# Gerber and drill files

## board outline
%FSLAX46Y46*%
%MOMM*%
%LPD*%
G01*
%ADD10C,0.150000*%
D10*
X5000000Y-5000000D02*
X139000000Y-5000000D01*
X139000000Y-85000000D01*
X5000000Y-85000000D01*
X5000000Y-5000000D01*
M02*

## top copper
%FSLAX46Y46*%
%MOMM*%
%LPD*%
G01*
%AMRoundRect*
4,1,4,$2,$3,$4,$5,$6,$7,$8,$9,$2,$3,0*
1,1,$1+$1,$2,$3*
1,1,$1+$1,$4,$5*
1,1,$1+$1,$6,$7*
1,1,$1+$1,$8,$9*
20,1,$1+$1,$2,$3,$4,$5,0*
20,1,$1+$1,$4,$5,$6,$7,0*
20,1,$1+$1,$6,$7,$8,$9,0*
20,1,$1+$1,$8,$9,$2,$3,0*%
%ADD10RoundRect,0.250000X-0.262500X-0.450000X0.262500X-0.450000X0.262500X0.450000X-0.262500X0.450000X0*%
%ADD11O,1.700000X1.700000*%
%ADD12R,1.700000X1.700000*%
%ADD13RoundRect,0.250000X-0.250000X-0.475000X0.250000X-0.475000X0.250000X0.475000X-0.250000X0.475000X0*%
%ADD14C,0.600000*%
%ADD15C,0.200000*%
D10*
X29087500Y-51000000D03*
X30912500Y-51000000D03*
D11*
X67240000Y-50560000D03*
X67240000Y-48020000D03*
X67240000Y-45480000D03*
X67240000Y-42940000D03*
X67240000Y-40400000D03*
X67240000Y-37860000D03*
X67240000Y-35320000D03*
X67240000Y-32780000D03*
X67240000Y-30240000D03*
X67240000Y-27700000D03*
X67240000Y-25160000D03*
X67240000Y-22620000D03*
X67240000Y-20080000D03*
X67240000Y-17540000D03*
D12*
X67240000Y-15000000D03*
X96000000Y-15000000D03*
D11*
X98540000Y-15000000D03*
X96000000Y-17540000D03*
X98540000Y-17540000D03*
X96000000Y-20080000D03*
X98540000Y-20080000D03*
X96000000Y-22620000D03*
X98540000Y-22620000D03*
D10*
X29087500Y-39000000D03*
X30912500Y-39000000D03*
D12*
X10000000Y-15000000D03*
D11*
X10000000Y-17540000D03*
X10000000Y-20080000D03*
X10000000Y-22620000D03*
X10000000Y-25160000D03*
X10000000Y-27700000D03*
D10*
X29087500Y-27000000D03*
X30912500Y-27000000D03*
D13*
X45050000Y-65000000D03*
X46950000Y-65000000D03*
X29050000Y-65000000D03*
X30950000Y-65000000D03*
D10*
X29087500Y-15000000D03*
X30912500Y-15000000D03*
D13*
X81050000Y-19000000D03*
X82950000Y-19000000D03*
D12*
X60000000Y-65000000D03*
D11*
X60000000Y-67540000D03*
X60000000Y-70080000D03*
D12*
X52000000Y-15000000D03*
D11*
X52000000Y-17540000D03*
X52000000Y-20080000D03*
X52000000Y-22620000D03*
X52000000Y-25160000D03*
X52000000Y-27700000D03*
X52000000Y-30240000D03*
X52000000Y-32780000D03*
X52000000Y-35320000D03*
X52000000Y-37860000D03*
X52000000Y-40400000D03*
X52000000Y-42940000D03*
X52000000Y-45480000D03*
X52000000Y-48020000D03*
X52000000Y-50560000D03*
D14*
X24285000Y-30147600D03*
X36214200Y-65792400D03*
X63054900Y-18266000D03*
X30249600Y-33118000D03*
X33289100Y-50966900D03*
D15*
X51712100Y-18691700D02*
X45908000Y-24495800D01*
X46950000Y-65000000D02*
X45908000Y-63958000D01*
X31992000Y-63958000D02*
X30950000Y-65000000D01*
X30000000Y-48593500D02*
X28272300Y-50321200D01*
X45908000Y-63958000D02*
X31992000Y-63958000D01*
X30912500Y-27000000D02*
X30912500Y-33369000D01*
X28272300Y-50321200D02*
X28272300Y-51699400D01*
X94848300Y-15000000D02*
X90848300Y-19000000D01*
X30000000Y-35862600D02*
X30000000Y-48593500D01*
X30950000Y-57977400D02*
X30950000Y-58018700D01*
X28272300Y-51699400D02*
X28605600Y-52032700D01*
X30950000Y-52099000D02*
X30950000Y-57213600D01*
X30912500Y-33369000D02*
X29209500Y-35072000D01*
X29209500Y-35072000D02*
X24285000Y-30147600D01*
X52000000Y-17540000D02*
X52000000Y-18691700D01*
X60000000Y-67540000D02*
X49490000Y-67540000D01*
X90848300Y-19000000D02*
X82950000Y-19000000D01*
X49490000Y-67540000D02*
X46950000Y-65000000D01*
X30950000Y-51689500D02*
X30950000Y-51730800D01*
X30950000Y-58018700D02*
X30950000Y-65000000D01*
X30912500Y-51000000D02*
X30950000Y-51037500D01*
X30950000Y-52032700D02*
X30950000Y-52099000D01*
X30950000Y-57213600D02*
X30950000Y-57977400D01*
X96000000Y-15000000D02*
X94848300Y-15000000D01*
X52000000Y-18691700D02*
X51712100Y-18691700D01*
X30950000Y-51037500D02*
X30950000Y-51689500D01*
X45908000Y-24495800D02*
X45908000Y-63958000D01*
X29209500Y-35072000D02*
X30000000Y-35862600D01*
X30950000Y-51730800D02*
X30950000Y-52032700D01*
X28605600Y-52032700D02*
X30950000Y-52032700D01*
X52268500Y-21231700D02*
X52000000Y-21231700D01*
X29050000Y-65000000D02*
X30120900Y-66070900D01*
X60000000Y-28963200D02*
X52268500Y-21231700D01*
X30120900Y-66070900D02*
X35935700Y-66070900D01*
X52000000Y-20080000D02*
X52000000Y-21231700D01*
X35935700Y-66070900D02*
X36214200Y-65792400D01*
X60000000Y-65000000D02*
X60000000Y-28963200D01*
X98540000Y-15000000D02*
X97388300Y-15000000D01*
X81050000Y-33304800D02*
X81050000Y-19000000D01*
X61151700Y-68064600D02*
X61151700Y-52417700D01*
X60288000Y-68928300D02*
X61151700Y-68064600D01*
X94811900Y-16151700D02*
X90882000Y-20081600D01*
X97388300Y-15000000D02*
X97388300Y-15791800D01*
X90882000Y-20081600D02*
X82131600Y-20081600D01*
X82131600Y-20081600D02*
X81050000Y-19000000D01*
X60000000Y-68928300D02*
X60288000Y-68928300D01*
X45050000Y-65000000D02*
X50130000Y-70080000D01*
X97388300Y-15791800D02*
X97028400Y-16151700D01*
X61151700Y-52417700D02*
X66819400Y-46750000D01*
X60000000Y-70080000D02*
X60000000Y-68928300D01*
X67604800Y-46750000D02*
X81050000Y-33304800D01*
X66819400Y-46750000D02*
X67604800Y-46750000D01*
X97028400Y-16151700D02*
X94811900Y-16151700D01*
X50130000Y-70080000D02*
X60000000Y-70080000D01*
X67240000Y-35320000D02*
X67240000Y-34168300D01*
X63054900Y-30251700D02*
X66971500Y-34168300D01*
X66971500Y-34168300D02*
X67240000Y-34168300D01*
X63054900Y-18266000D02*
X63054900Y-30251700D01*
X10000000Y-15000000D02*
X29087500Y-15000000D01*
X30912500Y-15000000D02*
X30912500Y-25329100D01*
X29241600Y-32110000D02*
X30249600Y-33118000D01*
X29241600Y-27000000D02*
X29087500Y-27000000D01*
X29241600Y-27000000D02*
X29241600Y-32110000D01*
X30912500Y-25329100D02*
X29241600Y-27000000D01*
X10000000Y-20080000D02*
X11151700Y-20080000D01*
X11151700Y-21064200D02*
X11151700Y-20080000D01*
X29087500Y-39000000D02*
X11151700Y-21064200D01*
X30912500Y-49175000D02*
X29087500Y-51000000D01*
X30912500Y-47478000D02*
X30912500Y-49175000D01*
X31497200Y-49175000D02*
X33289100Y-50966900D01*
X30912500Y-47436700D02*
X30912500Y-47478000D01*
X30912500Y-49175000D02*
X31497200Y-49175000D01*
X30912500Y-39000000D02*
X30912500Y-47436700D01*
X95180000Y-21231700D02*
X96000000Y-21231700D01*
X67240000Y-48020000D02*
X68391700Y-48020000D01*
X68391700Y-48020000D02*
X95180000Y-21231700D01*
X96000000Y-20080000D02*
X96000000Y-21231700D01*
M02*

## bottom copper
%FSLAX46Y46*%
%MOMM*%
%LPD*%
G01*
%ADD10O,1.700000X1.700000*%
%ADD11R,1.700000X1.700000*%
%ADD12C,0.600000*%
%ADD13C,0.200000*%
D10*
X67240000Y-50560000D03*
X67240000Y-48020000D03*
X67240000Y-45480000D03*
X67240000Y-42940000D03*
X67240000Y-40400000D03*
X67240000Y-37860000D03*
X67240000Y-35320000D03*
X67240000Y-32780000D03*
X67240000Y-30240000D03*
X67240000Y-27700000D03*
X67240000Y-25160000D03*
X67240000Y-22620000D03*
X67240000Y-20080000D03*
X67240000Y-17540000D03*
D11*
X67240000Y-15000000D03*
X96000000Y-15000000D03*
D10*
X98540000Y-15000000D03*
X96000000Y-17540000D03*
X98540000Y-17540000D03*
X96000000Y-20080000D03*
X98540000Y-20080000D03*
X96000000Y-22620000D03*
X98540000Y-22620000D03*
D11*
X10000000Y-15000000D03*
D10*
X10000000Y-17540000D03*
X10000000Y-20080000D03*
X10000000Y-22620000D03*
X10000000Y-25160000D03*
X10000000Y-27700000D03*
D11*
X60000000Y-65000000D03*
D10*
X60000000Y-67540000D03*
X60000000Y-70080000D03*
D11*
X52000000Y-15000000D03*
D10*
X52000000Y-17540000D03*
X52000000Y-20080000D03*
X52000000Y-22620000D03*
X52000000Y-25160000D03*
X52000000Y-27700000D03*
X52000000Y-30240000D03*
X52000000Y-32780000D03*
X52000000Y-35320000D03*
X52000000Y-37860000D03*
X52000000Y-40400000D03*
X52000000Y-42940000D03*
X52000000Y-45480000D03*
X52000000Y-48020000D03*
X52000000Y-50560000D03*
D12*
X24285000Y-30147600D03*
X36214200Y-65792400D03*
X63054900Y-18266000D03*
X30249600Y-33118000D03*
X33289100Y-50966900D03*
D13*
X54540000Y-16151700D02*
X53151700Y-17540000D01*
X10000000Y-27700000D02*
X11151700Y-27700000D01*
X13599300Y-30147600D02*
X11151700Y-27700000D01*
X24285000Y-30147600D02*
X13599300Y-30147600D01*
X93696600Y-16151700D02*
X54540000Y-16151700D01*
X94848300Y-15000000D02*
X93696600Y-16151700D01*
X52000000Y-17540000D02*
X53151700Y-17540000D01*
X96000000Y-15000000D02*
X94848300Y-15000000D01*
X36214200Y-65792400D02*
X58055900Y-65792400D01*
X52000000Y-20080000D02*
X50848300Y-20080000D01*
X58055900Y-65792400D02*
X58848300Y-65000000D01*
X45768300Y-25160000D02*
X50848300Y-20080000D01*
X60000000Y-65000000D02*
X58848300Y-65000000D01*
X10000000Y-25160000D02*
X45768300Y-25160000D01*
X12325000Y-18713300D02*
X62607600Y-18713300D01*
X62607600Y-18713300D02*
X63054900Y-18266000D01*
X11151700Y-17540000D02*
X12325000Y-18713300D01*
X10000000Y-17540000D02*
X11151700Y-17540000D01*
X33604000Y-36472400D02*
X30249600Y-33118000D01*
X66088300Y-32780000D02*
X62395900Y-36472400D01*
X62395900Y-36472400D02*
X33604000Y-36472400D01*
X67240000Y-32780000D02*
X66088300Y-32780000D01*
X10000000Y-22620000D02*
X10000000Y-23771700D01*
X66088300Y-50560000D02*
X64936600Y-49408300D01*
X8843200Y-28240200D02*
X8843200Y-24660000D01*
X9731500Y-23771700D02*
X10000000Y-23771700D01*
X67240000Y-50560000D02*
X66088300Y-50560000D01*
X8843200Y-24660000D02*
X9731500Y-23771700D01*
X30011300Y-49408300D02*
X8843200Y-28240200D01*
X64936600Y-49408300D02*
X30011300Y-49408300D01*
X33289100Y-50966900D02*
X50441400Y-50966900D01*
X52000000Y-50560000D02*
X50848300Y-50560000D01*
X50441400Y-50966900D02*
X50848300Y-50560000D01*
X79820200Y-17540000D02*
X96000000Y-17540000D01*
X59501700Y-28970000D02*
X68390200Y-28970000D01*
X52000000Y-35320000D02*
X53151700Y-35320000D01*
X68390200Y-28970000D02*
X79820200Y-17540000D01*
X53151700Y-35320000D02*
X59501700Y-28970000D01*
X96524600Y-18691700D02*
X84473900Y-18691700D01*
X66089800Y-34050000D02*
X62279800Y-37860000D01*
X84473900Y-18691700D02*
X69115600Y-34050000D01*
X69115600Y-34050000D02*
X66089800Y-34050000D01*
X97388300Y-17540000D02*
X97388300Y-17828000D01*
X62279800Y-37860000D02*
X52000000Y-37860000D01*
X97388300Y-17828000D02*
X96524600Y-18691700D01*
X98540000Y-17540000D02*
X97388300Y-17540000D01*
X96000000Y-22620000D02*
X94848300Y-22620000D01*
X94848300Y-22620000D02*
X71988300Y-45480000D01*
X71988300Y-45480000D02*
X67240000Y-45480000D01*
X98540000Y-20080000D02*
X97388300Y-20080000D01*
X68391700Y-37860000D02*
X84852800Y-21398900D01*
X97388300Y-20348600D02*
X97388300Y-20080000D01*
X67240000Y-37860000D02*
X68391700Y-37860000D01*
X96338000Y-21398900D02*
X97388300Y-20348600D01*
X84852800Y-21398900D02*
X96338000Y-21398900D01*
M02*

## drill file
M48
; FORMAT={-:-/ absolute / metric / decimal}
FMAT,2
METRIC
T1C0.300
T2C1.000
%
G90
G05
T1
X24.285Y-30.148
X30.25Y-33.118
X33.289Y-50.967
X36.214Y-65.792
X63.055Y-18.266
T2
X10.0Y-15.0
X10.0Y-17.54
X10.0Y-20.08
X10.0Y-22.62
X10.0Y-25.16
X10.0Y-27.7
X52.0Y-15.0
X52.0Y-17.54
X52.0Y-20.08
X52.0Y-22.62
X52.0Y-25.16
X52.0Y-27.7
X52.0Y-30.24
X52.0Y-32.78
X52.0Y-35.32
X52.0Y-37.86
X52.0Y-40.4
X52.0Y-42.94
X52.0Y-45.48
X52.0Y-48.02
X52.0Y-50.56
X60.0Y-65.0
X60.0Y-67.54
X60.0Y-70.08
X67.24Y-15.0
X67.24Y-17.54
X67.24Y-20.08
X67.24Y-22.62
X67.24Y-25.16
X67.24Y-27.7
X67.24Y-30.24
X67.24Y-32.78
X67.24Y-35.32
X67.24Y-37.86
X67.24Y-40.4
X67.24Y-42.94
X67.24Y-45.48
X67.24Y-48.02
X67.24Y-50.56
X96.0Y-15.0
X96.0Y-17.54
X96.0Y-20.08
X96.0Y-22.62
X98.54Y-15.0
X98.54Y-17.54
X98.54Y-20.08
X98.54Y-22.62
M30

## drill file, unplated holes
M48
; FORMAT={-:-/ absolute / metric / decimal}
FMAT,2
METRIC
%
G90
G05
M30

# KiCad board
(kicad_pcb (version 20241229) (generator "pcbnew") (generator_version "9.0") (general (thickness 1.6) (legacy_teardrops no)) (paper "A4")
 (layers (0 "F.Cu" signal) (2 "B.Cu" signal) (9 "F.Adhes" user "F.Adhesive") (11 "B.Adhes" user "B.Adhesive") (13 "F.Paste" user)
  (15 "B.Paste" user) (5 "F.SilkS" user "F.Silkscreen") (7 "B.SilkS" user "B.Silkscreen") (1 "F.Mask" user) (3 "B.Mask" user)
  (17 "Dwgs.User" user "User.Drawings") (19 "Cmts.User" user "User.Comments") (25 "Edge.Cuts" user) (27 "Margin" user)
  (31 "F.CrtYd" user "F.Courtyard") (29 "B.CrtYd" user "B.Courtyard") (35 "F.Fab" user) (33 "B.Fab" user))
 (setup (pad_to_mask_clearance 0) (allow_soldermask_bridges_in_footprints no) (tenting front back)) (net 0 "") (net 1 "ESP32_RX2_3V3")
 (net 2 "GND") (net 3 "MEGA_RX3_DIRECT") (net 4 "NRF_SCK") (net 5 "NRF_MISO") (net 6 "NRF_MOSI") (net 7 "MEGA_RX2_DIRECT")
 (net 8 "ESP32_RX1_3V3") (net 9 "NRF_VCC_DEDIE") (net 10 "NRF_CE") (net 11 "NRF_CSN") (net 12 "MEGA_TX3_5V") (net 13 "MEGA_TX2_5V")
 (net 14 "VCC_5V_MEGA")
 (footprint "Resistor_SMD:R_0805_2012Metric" (layer "F.Cu") (at 30 51)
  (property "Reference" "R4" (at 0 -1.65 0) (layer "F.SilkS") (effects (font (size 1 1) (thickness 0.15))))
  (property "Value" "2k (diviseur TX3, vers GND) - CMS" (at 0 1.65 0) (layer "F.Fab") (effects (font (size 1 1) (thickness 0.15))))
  (pad "1" smd roundrect (at -0.9125 0) (size 1.025 1.4) (layers "F.Cu" "F.Mask" "F.Paste") (roundrect_rratio 0.243902)
   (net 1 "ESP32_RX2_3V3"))
  (pad "2" smd roundrect (at 0.9125 0) (size 1.025 1.4) (layers "F.Cu" "F.Mask" "F.Paste") (roundrect_rratio 0.243902) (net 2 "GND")))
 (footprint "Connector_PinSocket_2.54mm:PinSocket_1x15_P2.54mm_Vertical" (layer "F.Cu") (at 67.24 15)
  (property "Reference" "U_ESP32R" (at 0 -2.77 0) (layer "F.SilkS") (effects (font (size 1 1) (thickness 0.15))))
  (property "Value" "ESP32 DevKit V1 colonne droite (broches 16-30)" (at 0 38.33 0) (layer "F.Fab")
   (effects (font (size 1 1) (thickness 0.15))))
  (pad "16" thru_hole oval (at 0 35.56) (size 1.7 1.7) (drill 1) (layers "*.Cu" "*.Mask") (remove_unused_layers no)
   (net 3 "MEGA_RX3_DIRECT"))
  (pad "17" thru_hole oval (at 0 33.02) (size 1.7 1.7) (drill 1) (layers "*.Cu" "*.Mask") (remove_unused_layers no) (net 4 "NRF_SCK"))
  (pad "18" thru_hole oval (at 0 30.48) (size 1.7 1.7) (drill 1) (layers "*.Cu" "*.Mask") (remove_unused_layers no) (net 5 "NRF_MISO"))
  (pad "19" thru_hole oval (at 0 27.94) (size 1.7 1.7) (drill 1) (layers "*.Cu" "*.Mask") (remove_unused_layers no))
  (pad "20" thru_hole oval (at 0 25.4) (size 1.7 1.7) (drill 1) (layers "*.Cu" "*.Mask") (remove_unused_layers no))
  (pad "21" thru_hole oval (at 0 22.86) (size 1.7 1.7) (drill 1) (layers "*.Cu" "*.Mask") (remove_unused_layers no) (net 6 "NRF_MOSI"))
  (pad "22" thru_hole oval (at 0 20.32) (size 1.7 1.7) (drill 1) (layers "*.Cu" "*.Mask") (remove_unused_layers no)
   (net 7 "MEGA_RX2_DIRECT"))
  (pad "23" thru_hole oval (at 0 17.78) (size 1.7 1.7) (drill 1) (layers "*.Cu" "*.Mask") (remove_unused_layers no) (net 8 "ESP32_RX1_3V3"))
  (pad "24" thru_hole oval (at 0 15.24) (size 1.7 1.7) (drill 1) (layers "*.Cu" "*.Mask") (remove_unused_layers no))
  (pad "25" thru_hole oval (at 0 12.7) (size 1.7 1.7) (drill 1) (layers "*.Cu" "*.Mask") (remove_unused_layers no))
  (pad "26" thru_hole oval (at 0 10.16) (size 1.7 1.7) (drill 1) (layers "*.Cu" "*.Mask") (remove_unused_layers no))
  (pad "27" thru_hole oval (at 0 7.62) (size 1.7 1.7) (drill 1) (layers "*.Cu" "*.Mask") (remove_unused_layers no))
  (pad "28" thru_hole oval (at 0 5.08) (size 1.7 1.7) (drill 1) (layers "*.Cu" "*.Mask") (remove_unused_layers no))
  (pad "29" thru_hole oval (at 0 2.54) (size 1.7 1.7) (drill 1) (layers "*.Cu" "*.Mask") (remove_unused_layers no))
  (pad "30" thru_hole rect (at 0 0) (size 1.7 1.7) (drill 1) (layers "*.Cu" "*.Mask") (remove_unused_layers no)))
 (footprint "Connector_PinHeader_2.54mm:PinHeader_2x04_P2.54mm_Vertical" (layer "F.Cu") (at 96 15)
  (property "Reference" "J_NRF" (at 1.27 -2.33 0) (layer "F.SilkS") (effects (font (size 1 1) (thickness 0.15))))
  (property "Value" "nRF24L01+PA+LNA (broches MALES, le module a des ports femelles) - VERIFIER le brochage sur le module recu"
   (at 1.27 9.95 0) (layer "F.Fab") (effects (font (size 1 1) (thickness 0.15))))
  (pad "1" thru_hole rect (at 0 0) (size 1.7 1.7) (drill 1) (layers "*.Cu" "*.Mask") (remove_unused_layers no) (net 2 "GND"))
  (pad "2" thru_hole oval (at 2.54 0) (size 1.7 1.7) (drill 1) (layers "*.Cu" "*.Mask") (remove_unused_layers no) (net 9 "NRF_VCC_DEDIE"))
  (pad "3" thru_hole oval (at 0 2.54) (size 1.7 1.7) (drill 1) (layers "*.Cu" "*.Mask") (remove_unused_layers no) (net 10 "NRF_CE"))
  (pad "4" thru_hole oval (at 2.54 2.54) (size 1.7 1.7) (drill 1) (layers "*.Cu" "*.Mask") (remove_unused_layers no) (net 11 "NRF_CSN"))
  (pad "5" thru_hole oval (at 0 5.08) (size 1.7 1.7) (drill 1) (layers "*.Cu" "*.Mask") (remove_unused_layers no) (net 4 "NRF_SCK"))
  (pad "6" thru_hole oval (at 2.54 5.08) (size 1.7 1.7) (drill 1) (layers "*.Cu" "*.Mask") (remove_unused_layers no) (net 6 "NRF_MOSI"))
  (pad "7" thru_hole oval (at 0 7.62) (size 1.7 1.7) (drill 1) (layers "*.Cu" "*.Mask") (remove_unused_layers no) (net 5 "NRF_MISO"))
  (pad "8" thru_hole oval (at 2.54 7.62) (size 1.7 1.7) (drill 1) (layers "*.Cu" "*.Mask") (remove_unused_layers no)))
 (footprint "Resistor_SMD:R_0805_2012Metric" (layer "F.Cu") (at 30 39)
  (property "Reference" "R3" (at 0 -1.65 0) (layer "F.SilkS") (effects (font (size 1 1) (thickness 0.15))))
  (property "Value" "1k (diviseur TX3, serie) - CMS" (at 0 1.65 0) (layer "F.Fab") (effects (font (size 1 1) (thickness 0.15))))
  (pad "1" smd roundrect (at -0.9125 0) (size 1.025 1.4) (layers "F.Cu" "F.Mask" "F.Paste") (roundrect_rratio 0.243902)
   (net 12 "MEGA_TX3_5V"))
  (pad "2" smd roundrect (at 0.9125 0) (size 1.025 1.4) (layers "F.Cu" "F.Mask" "F.Paste") (roundrect_rratio 0.243902)
   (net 1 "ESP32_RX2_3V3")))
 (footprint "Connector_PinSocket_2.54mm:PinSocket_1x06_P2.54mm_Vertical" (layer "F.Cu") (at 10 15)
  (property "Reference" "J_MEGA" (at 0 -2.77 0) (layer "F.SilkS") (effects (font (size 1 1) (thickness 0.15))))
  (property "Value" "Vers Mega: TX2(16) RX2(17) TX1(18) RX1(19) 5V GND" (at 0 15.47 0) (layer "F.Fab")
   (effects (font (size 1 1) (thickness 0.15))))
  (pad "1" thru_hole rect (at 0 0) (size 1.7 1.7) (drill 1) (layers "*.Cu" "*.Mask") (remove_unused_layers no) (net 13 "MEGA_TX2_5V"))
  (pad "2" thru_hole oval (at 0 2.54) (size 1.7 1.7) (drill 1) (layers "*.Cu" "*.Mask") (remove_unused_layers no) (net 7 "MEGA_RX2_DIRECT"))
  (pad "3" thru_hole oval (at 0 5.08) (size 1.7 1.7) (drill 1) (layers "*.Cu" "*.Mask") (remove_unused_layers no) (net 12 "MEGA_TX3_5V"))
  (pad "4" thru_hole oval (at 0 7.62) (size 1.7 1.7) (drill 1) (layers "*.Cu" "*.Mask") (remove_unused_layers no) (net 3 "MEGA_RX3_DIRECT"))
  (pad "5" thru_hole oval (at 0 10.16) (size 1.7 1.7) (drill 1) (layers "*.Cu" "*.Mask") (remove_unused_layers no) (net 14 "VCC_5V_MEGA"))
  (pad "6" thru_hole oval (at 0 12.7) (size 1.7 1.7) (drill 1) (layers "*.Cu" "*.Mask") (remove_unused_layers no) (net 2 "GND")))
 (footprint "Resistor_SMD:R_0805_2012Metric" (layer "F.Cu") (at 30 27)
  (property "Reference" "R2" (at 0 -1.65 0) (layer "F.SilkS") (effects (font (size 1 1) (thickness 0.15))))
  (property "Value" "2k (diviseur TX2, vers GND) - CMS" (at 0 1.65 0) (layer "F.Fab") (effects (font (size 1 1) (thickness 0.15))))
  (pad "1" smd roundrect (at -0.9125 0) (size 1.025 1.4) (layers "F.Cu" "F.Mask" "F.Paste") (roundrect_rratio 0.243902)
   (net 8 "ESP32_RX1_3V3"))
  (pad "2" smd roundrect (at 0.9125 0) (size 1.025 1.4) (layers "F.Cu" "F.Mask" "F.Paste") (roundrect_rratio 0.243902) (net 2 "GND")))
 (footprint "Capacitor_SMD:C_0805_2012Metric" (layer "F.Cu") (at 46 65)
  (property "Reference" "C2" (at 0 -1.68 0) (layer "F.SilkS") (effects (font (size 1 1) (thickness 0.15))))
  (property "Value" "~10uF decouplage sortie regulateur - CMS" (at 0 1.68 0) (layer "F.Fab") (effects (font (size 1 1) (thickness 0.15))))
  (pad "1" smd roundrect (at -0.95 0) (size 1 1.45) (layers "F.Cu" "F.Mask" "F.Paste") (roundrect_rratio 0.25) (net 9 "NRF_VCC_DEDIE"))
  (pad "2" smd roundrect (at 0.95 0) (size 1 1.45) (layers "F.Cu" "F.Mask" "F.Paste") (roundrect_rratio 0.25) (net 2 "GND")))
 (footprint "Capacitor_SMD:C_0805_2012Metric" (layer "F.Cu") (at 30 65)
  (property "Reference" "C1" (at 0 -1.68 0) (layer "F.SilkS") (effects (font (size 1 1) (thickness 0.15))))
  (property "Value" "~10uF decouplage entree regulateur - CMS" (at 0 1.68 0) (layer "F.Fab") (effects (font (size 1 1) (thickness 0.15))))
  (pad "1" smd roundrect (at -0.95 0) (size 1 1.45) (layers "F.Cu" "F.Mask" "F.Paste") (roundrect_rratio 0.25) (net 14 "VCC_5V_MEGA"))
  (pad "2" smd roundrect (at 0.95 0) (size 1 1.45) (layers "F.Cu" "F.Mask" "F.Paste") (roundrect_rratio 0.25) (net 2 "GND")))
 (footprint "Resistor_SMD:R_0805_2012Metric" (layer "F.Cu") (at 30 15)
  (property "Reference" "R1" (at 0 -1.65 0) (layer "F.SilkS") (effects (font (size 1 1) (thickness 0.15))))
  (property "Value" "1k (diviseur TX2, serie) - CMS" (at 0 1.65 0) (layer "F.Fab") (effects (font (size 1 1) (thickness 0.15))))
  (pad "1" smd roundrect (at -0.9125 0) (size 1.025 1.4) (layers "F.Cu" "F.Mask" "F.Paste") (roundrect_rratio 0.243902)
   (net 13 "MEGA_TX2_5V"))
  (pad "2" smd roundrect (at 0.9125 0) (size 1.025 1.4) (layers "F.Cu" "F.Mask" "F.Paste") (roundrect_rratio 0.243902)
   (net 8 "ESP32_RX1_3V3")))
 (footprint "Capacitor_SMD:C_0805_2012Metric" (layer "F.Cu") (at 82 19)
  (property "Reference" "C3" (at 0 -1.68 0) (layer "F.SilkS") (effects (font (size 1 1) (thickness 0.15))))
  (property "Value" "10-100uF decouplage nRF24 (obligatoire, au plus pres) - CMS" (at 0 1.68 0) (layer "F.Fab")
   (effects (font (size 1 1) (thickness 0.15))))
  (pad "1" smd roundrect (at -0.95 0) (size 1 1.45) (layers "F.Cu" "F.Mask" "F.Paste") (roundrect_rratio 0.25) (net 9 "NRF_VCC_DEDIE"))
  (pad "2" smd roundrect (at 0.95 0) (size 1 1.45) (layers "F.Cu" "F.Mask" "F.Paste") (roundrect_rratio 0.25) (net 2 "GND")))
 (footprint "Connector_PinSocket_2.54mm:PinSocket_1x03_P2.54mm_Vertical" (layer "F.Cu") (at 60 65)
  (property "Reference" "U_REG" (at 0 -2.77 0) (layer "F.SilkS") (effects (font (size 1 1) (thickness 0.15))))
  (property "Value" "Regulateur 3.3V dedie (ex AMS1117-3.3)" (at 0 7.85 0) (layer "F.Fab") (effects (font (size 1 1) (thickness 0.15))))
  (pad "1" thru_hole rect (at 0 0) (size 1.7 1.7) (drill 1) (layers "*.Cu" "*.Mask") (remove_unused_layers no) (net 14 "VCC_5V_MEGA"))
  (pad "2" thru_hole oval (at 0 2.54) (size 1.7 1.7) (drill 1) (layers "*.Cu" "*.Mask") (remove_unused_layers no) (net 2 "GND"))
  (pad "3" thru_hole oval (at 0 5.08) (size 1.7 1.7) (drill 1) (layers "*.Cu" "*.Mask") (remove_unused_layers no) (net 9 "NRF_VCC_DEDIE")))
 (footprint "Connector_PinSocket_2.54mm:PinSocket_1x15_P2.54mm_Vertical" (layer "F.Cu") (at 52 15)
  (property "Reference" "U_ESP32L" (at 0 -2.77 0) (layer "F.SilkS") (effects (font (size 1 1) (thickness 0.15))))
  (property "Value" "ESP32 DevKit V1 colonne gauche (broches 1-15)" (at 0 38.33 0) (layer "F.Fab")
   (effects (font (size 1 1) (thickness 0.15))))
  (pad "1" thru_hole rect (at 0 0) (size 1.7 1.7) (drill 1) (layers "*.Cu" "*.Mask") (remove_unused_layers no))
  (pad "2" thru_hole oval (at 0 2.54) (size 1.7 1.7) (drill 1) (layers "*.Cu" "*.Mask") (remove_unused_layers no) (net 2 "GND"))
  (pad "3" thru_hole oval (at 0 5.08) (size 1.7 1.7) (drill 1) (layers "*.Cu" "*.Mask") (remove_unused_layers no) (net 14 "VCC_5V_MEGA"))
  (pad "4" thru_hole oval (at 0 7.62) (size 1.7 1.7) (drill 1) (layers "*.Cu" "*.Mask") (remove_unused_layers no))
  (pad "5" thru_hole oval (at 0 10.16) (size 1.7 1.7) (drill 1) (layers "*.Cu" "*.Mask") (remove_unused_layers no))
  (pad "6" thru_hole oval (at 0 12.7) (size 1.7 1.7) (drill 1) (layers "*.Cu" "*.Mask") (remove_unused_layers no))
  (pad "7" thru_hole oval (at 0 15.24) (size 1.7 1.7) (drill 1) (layers "*.Cu" "*.Mask") (remove_unused_layers no))
  (pad "8" thru_hole oval (at 0 17.78) (size 1.7 1.7) (drill 1) (layers "*.Cu" "*.Mask") (remove_unused_layers no))
  (pad "9" thru_hole oval (at 0 20.32) (size 1.7 1.7) (drill 1) (layers "*.Cu" "*.Mask") (remove_unused_layers no) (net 10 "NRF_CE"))
  (pad "10" thru_hole oval (at 0 22.86) (size 1.7 1.7) (drill 1) (layers "*.Cu" "*.Mask") (remove_unused_layers no) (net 11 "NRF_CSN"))
  (pad "11" thru_hole oval (at 0 25.4) (size 1.7 1.7) (drill 1) (layers "*.Cu" "*.Mask") (remove_unused_layers no))
  (pad "12" thru_hole oval (at 0 27.94) (size 1.7 1.7) (drill 1) (layers "*.Cu" "*.Mask") (remove_unused_layers no))
  (pad "13" thru_hole oval (at 0 30.48) (size 1.7 1.7) (drill 1) (layers "*.Cu" "*.Mask") (remove_unused_layers no))
  (pad "14" thru_hole oval (at 0 33.02) (size 1.7 1.7) (drill 1) (layers "*.Cu" "*.Mask") (remove_unused_layers no))
  (pad "15" thru_hole oval (at 0 35.56) (size 1.7 1.7) (drill 1) (layers "*.Cu" "*.Mask") (remove_unused_layers no) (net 1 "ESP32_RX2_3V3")))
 (gr_rect (start 5 5) (end 139 85) (stroke (width 0.15) (type default)) (fill no) (layer "Edge.Cuts"))
 (segment (start 51.7121 18.6917) (end 45.908 24.4958) (width 0.2) (layer "F.Cu") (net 2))
 (segment (start 46.95 65) (end 45.908 63.958) (width 0.2) (layer "F.Cu") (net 2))
 (segment (start 31.992 63.958) (end 30.95 65) (width 0.2) (layer "F.Cu") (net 2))
 (segment (start 30 48.5935) (end 28.2723 50.3212) (width 0.2) (layer "F.Cu") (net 2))
 (segment (start 45.908 63.958) (end 31.992 63.958) (width 0.2) (layer "F.Cu") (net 2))
 (segment (start 30.9125 27) (end 30.9125 33.369) (width 0.2) (layer "F.Cu") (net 2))
 (segment (start 28.2723 50.3212) (end 28.2723 51.6994) (width 0.2) (layer "F.Cu") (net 2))
 (segment (start 94.8483 15) (end 90.8483 19) (width 0.2) (layer "F.Cu") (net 2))
 (segment (start 30 35.8626) (end 30 48.5935) (width 0.2) (layer "F.Cu") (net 2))
 (segment (start 30.95 57.9774) (end 30.95 58.0187) (width 0.2) (layer "F.Cu") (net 2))
 (segment (start 28.2723 51.6994) (end 28.6056 52.0327) (width 0.2) (layer "F.Cu") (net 2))
 (segment (start 30.95 52.099) (end 30.95 57.2136) (width 0.2) (layer "F.Cu") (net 2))
 (segment (start 30.9125 33.369) (end 29.2095 35.072) (width 0.2) (layer "F.Cu") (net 2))
 (segment (start 29.2095 35.072) (end 24.285 30.1476) (width 0.2) (layer "F.Cu") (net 2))
 (segment (start 52 17.54) (end 52 18.6917) (width 0.2) (layer "F.Cu") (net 2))
 (segment (start 60 67.54) (end 49.49 67.54) (width 0.2) (layer "F.Cu") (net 2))
 (segment (start 90.8483 19) (end 82.95 19) (width 0.2) (layer "F.Cu") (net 2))
 (segment (start 49.49 67.54) (end 46.95 65) (width 0.2) (layer "F.Cu") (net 2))
 (segment (start 30.95 51.6895) (end 30.95 51.7308) (width 0.2) (layer "F.Cu") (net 2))
 (segment (start 30.95 58.0187) (end 30.95 65) (width 0.2) (layer "F.Cu") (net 2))
 (segment (start 30.9125 51) (end 30.95 51.0375) (width 0.2) (layer "F.Cu") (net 2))
 (segment (start 30.95 52.0327) (end 30.95 52.099) (width 0.2) (layer "F.Cu") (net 2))
 (segment (start 30.95 57.2136) (end 30.95 57.9774) (width 0.2) (layer "F.Cu") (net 2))
 (segment (start 96 15) (end 94.8483 15) (width 0.2) (layer "F.Cu") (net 2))
 (segment (start 52 18.6917) (end 51.7121 18.6917) (width 0.2) (layer "F.Cu") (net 2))
 (segment (start 30.95 51.0375) (end 30.95 51.6895) (width 0.2) (layer "F.Cu") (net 2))
 (segment (start 45.908 24.4958) (end 45.908 63.958) (width 0.2) (layer "F.Cu") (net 2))
 (segment (start 29.2095 35.072) (end 30 35.8626) (width 0.2) (layer "F.Cu") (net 2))
 (segment (start 30.95 51.7308) (end 30.95 52.0327) (width 0.2) (layer "F.Cu") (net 2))
 (segment (start 28.6056 52.0327) (end 30.95 52.0327) (width 0.2) (layer "F.Cu") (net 2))
 (via (at 24.285 30.1476) (size 0.6) (drill 0.3) (layers "F.Cu" "B.Cu") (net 2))
 (segment (start 54.54 16.1517) (end 53.1517 17.54) (width 0.2) (layer "B.Cu") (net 2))
 (segment (start 10 27.7) (end 11.1517 27.7) (width 0.2) (layer "B.Cu") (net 2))
 (segment (start 13.5993 30.1476) (end 11.1517 27.7) (width 0.2) (layer "B.Cu") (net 2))
 (segment (start 24.285 30.1476) (end 13.5993 30.1476) (width 0.2) (layer "B.Cu") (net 2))
 (segment (start 93.6966 16.1517) (end 54.54 16.1517) (width 0.2) (layer "B.Cu") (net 2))
 (segment (start 94.8483 15) (end 93.6966 16.1517) (width 0.2) (layer "B.Cu") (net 2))
 (segment (start 52 17.54) (end 53.1517 17.54) (width 0.2) (layer "B.Cu") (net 2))
 (segment (start 96 15) (end 94.8483 15) (width 0.2) (layer "B.Cu") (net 2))
 (segment (start 52.2685 21.2317) (end 52 21.2317) (width 0.2) (layer "F.Cu") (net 14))
 (segment (start 29.05 65) (end 30.1209 66.0709) (width 0.2) (layer "F.Cu") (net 14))
 (segment (start 60 28.9632) (end 52.2685 21.2317) (width 0.2) (layer "F.Cu") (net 14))
 (segment (start 30.1209 66.0709) (end 35.9357 66.0709) (width 0.2) (layer "F.Cu") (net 14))
 (segment (start 52 20.08) (end 52 21.2317) (width 0.2) (layer "F.Cu") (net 14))
 (segment (start 35.9357 66.0709) (end 36.2142 65.7924) (width 0.2) (layer "F.Cu") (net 14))
 (segment (start 60 65) (end 60 28.9632) (width 0.2) (layer "F.Cu") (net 14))
 (via (at 36.2142 65.7924) (size 0.6) (drill 0.3) (layers "F.Cu" "B.Cu") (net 14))
 (segment (start 36.2142 65.7924) (end 58.0559 65.7924) (width 0.2) (layer "B.Cu") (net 14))
 (segment (start 52 20.08) (end 50.8483 20.08) (width 0.2) (layer "B.Cu") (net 14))
 (segment (start 58.0559 65.7924) (end 58.8483 65) (width 0.2) (layer "B.Cu") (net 14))
 (segment (start 45.7683 25.16) (end 50.8483 20.08) (width 0.2) (layer "B.Cu") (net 14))
 (segment (start 60 65) (end 58.8483 65) (width 0.2) (layer "B.Cu") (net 14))
 (segment (start 10 25.16) (end 45.7683 25.16) (width 0.2) (layer "B.Cu") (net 14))
 (segment (start 98.54 15) (end 97.3883 15) (width 0.2) (layer "F.Cu") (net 9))
 (segment (start 81.05 33.3048) (end 81.05 19) (width 0.2) (layer "F.Cu") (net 9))
 (segment (start 61.1517 68.0646) (end 61.1517 52.4177) (width 0.2) (layer "F.Cu") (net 9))
 (segment (start 60.288 68.9283) (end 61.1517 68.0646) (width 0.2) (layer "F.Cu") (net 9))
 (segment (start 94.8119 16.1517) (end 90.882 20.0816) (width 0.2) (layer "F.Cu") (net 9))
 (segment (start 97.3883 15) (end 97.3883 15.7918) (width 0.2) (layer "F.Cu") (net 9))
 (segment (start 90.882 20.0816) (end 82.1316 20.0816) (width 0.2) (layer "F.Cu") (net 9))
 (segment (start 82.1316 20.0816) (end 81.05 19) (width 0.2) (layer "F.Cu") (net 9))
 (segment (start 60 68.9283) (end 60.288 68.9283) (width 0.2) (layer "F.Cu") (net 9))
 (segment (start 45.05 65) (end 50.13 70.08) (width 0.2) (layer "F.Cu") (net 9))
 (segment (start 97.3883 15.7918) (end 97.0284 16.1517) (width 0.2) (layer "F.Cu") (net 9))
 (segment (start 61.1517 52.4177) (end 66.8194 46.75) (width 0.2) (layer "F.Cu") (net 9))
 (segment (start 60 70.08) (end 60 68.9283) (width 0.2) (layer "F.Cu") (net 9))
 (segment (start 67.6048 46.75) (end 81.05 33.3048) (width 0.2) (layer "F.Cu") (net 9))
 (segment (start 66.8194 46.75) (end 67.6048 46.75) (width 0.2) (layer "F.Cu") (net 9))
 (segment (start 97.0284 16.1517) (end 94.8119 16.1517) (width 0.2) (layer "F.Cu") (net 9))
 (segment (start 50.13 70.08) (end 60 70.08) (width 0.2) (layer "F.Cu") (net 9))
 (segment (start 67.24 35.32) (end 67.24 34.1683) (width 0.2) (layer "F.Cu") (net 7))
 (segment (start 63.0549 30.2517) (end 66.9715 34.1683) (width 0.2) (layer "F.Cu") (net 7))
 (segment (start 66.9715 34.1683) (end 67.24 34.1683) (width 0.2) (layer "F.Cu") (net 7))
 (segment (start 63.0549 18.266) (end 63.0549 30.2517) (width 0.2) (layer "F.Cu") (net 7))
 (via (at 63.0549 18.266) (size 0.6) (drill 0.3) (layers "F.Cu" "B.Cu") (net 7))
 (segment (start 12.325 18.7133) (end 62.6076 18.7133) (width 0.2) (layer "B.Cu") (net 7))
 (segment (start 62.6076 18.7133) (end 63.0549 18.266) (width 0.2) (layer "B.Cu") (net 7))
 (segment (start 11.1517 17.54) (end 12.325 18.7133) (width 0.2) (layer "B.Cu") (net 7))
 (segment (start 10 17.54) (end 11.1517 17.54) (width 0.2) (layer "B.Cu") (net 7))
 (segment (start 10 15) (end 29.0875 15) (width 0.2) (layer "F.Cu") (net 13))
 (segment (start 30.9125 15) (end 30.9125 25.3291) (width 0.2) (layer "F.Cu") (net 8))
 (segment (start 29.2416 32.11) (end 30.2496 33.118) (width 0.2) (layer "F.Cu") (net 8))
 (segment (start 29.2416 27) (end 29.0875 27) (width 0.2) (layer "F.Cu") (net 8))
 (segment (start 29.2416 27) (end 29.2416 32.11) (width 0.2) (layer "F.Cu") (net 8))
 (segment (start 30.9125 25.3291) (end 29.2416 27) (width 0.2) (layer "F.Cu") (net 8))
 (via (at 30.2496 33.118) (size 0.6) (drill 0.3) (layers "F.Cu" "B.Cu") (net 8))
 (segment (start 33.604 36.4724) (end 30.2496 33.118) (width 0.2) (layer "B.Cu") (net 8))
 (segment (start 66.0883 32.78) (end 62.3959 36.4724) (width 0.2) (layer "B.Cu") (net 8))
 (segment (start 62.3959 36.4724) (end 33.604 36.4724) (width 0.2) (layer "B.Cu") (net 8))
 (segment (start 67.24 32.78) (end 66.0883 32.78) (width 0.2) (layer "B.Cu") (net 8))
 (segment (start 10 22.62) (end 10 23.7717) (width 0.2) (layer "B.Cu") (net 3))
 (segment (start 66.0883 50.56) (end 64.9366 49.4083) (width 0.2) (layer "B.Cu") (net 3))
 (segment (start 8.8432 28.2402) (end 8.8432 24.66) (width 0.2) (layer "B.Cu") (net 3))
 (segment (start 9.7315 23.7717) (end 10 23.7717) (width 0.2) (layer "B.Cu") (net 3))
 (segment (start 67.24 50.56) (end 66.0883 50.56) (width 0.2) (layer "B.Cu") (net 3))
 (segment (start 8.8432 24.66) (end 9.7315 23.7717) (width 0.2) (layer "B.Cu") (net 3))
 (segment (start 30.0113 49.4083) (end 8.8432 28.2402) (width 0.2) (layer "B.Cu") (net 3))
 (segment (start 64.9366 49.4083) (end 30.0113 49.4083) (width 0.2) (layer "B.Cu") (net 3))
 (segment (start 10 20.08) (end 11.1517 20.08) (width 0.2) (layer "F.Cu") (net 12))
 (segment (start 11.1517 21.0642) (end 11.1517 20.08) (width 0.2) (layer "F.Cu") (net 12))
 (segment (start 29.0875 39) (end 11.1517 21.0642) (width 0.2) (layer "F.Cu") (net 12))
 (segment (start 30.9125 49.175) (end 29.0875 51) (width 0.2) (layer "F.Cu") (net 1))
 (segment (start 30.9125 47.478) (end 30.9125 49.175) (width 0.2) (layer "F.Cu") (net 1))
 (segment (start 31.4972 49.175) (end 33.2891 50.9669) (width 0.2) (layer "F.Cu") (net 1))
 (segment (start 30.9125 47.4367) (end 30.9125 47.478) (width 0.2) (layer "F.Cu") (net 1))
 (segment (start 30.9125 49.175) (end 31.4972 49.175) (width 0.2) (layer "F.Cu") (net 1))
 (segment (start 30.9125 39) (end 30.9125 47.4367) (width 0.2) (layer "F.Cu") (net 1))
 (via (at 33.2891 50.9669) (size 0.6) (drill 0.3) (layers "F.Cu" "B.Cu") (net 1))
 (segment (start 33.2891 50.9669) (end 50.4414 50.9669) (width 0.2) (layer "B.Cu") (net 1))
 (segment (start 52 50.56) (end 50.8483 50.56) (width 0.2) (layer "B.Cu") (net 1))
 (segment (start 50.4414 50.9669) (end 50.8483 50.56) (width 0.2) (layer "B.Cu") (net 1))
 (segment (start 79.8202 17.54) (end 96 17.54) (width 0.2) (layer "B.Cu") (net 10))
 (segment (start 59.5017 28.97) (end 68.3902 28.97) (width 0.2) (layer "B.Cu") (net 10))
 (segment (start 52 35.32) (end 53.1517 35.32) (width 0.2) (layer "B.Cu") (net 10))
 (segment (start 68.3902 28.97) (end 79.8202 17.54) (width 0.2) (layer "B.Cu") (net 10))
 (segment (start 53.1517 35.32) (end 59.5017 28.97) (width 0.2) (layer "B.Cu") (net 10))
 (segment (start 96.5246 18.6917) (end 84.4739 18.6917) (width 0.2) (layer "B.Cu") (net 11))
 (segment (start 66.0898 34.05) (end 62.2798 37.86) (width 0.2) (layer "B.Cu") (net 11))
 (segment (start 84.4739 18.6917) (end 69.1156 34.05) (width 0.2) (layer "B.Cu") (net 11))
 (segment (start 69.1156 34.05) (end 66.0898 34.05) (width 0.2) (layer "B.Cu") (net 11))
 (segment (start 97.3883 17.54) (end 97.3883 17.828) (width 0.2) (layer "B.Cu") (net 11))
 (segment (start 62.2798 37.86) (end 52 37.86) (width 0.2) (layer "B.Cu") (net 11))
 (segment (start 97.3883 17.828) (end 96.5246 18.6917) (width 0.2) (layer "B.Cu") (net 11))
 (segment (start 98.54 17.54) (end 97.3883 17.54) (width 0.2) (layer "B.Cu") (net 11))
 (segment (start 95.18 21.2317) (end 96 21.2317) (width 0.2) (layer "F.Cu") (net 4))
 (segment (start 67.24 48.02) (end 68.3917 48.02) (width 0.2) (layer "F.Cu") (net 4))
 (segment (start 68.3917 48.02) (end 95.18 21.2317) (width 0.2) (layer "F.Cu") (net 4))
 (segment (start 96 20.08) (end 96 21.2317) (width 0.2) (layer "F.Cu") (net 4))
 (segment (start 96 22.62) (end 94.8483 22.62) (width 0.2) (layer "B.Cu") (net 5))
 (segment (start 94.8483 22.62) (end 71.9883 45.48) (width 0.2) (layer "B.Cu") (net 5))
 (segment (start 71.9883 45.48) (end 67.24 45.48) (width 0.2) (layer "B.Cu") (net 5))
 (segment (start 98.54 20.08) (end 97.3883 20.08) (width 0.2) (layer "B.Cu") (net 6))
 (segment (start 68.3917 37.86) (end 84.8528 21.3989) (width 0.2) (layer "B.Cu") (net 6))
 (segment (start 97.3883 20.3486) (end 97.3883 20.08) (width 0.2) (layer "B.Cu") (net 6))
 (segment (start 67.24 37.86) (end 68.3917 37.86) (width 0.2) (layer "B.Cu") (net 6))
 (segment (start 96.338 21.3989) (end 97.3883 20.3486) (width 0.2) (layer "B.Cu") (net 6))
 (segment (start 84.8528 21.3989) (end 96.338 21.3989) (width 0.2) (layer "B.Cu") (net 6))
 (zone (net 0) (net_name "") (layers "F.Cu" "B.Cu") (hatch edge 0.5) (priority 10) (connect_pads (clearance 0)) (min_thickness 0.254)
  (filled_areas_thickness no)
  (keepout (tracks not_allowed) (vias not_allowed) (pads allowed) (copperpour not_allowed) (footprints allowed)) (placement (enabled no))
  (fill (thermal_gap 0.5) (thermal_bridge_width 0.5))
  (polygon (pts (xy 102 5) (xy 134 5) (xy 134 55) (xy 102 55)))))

